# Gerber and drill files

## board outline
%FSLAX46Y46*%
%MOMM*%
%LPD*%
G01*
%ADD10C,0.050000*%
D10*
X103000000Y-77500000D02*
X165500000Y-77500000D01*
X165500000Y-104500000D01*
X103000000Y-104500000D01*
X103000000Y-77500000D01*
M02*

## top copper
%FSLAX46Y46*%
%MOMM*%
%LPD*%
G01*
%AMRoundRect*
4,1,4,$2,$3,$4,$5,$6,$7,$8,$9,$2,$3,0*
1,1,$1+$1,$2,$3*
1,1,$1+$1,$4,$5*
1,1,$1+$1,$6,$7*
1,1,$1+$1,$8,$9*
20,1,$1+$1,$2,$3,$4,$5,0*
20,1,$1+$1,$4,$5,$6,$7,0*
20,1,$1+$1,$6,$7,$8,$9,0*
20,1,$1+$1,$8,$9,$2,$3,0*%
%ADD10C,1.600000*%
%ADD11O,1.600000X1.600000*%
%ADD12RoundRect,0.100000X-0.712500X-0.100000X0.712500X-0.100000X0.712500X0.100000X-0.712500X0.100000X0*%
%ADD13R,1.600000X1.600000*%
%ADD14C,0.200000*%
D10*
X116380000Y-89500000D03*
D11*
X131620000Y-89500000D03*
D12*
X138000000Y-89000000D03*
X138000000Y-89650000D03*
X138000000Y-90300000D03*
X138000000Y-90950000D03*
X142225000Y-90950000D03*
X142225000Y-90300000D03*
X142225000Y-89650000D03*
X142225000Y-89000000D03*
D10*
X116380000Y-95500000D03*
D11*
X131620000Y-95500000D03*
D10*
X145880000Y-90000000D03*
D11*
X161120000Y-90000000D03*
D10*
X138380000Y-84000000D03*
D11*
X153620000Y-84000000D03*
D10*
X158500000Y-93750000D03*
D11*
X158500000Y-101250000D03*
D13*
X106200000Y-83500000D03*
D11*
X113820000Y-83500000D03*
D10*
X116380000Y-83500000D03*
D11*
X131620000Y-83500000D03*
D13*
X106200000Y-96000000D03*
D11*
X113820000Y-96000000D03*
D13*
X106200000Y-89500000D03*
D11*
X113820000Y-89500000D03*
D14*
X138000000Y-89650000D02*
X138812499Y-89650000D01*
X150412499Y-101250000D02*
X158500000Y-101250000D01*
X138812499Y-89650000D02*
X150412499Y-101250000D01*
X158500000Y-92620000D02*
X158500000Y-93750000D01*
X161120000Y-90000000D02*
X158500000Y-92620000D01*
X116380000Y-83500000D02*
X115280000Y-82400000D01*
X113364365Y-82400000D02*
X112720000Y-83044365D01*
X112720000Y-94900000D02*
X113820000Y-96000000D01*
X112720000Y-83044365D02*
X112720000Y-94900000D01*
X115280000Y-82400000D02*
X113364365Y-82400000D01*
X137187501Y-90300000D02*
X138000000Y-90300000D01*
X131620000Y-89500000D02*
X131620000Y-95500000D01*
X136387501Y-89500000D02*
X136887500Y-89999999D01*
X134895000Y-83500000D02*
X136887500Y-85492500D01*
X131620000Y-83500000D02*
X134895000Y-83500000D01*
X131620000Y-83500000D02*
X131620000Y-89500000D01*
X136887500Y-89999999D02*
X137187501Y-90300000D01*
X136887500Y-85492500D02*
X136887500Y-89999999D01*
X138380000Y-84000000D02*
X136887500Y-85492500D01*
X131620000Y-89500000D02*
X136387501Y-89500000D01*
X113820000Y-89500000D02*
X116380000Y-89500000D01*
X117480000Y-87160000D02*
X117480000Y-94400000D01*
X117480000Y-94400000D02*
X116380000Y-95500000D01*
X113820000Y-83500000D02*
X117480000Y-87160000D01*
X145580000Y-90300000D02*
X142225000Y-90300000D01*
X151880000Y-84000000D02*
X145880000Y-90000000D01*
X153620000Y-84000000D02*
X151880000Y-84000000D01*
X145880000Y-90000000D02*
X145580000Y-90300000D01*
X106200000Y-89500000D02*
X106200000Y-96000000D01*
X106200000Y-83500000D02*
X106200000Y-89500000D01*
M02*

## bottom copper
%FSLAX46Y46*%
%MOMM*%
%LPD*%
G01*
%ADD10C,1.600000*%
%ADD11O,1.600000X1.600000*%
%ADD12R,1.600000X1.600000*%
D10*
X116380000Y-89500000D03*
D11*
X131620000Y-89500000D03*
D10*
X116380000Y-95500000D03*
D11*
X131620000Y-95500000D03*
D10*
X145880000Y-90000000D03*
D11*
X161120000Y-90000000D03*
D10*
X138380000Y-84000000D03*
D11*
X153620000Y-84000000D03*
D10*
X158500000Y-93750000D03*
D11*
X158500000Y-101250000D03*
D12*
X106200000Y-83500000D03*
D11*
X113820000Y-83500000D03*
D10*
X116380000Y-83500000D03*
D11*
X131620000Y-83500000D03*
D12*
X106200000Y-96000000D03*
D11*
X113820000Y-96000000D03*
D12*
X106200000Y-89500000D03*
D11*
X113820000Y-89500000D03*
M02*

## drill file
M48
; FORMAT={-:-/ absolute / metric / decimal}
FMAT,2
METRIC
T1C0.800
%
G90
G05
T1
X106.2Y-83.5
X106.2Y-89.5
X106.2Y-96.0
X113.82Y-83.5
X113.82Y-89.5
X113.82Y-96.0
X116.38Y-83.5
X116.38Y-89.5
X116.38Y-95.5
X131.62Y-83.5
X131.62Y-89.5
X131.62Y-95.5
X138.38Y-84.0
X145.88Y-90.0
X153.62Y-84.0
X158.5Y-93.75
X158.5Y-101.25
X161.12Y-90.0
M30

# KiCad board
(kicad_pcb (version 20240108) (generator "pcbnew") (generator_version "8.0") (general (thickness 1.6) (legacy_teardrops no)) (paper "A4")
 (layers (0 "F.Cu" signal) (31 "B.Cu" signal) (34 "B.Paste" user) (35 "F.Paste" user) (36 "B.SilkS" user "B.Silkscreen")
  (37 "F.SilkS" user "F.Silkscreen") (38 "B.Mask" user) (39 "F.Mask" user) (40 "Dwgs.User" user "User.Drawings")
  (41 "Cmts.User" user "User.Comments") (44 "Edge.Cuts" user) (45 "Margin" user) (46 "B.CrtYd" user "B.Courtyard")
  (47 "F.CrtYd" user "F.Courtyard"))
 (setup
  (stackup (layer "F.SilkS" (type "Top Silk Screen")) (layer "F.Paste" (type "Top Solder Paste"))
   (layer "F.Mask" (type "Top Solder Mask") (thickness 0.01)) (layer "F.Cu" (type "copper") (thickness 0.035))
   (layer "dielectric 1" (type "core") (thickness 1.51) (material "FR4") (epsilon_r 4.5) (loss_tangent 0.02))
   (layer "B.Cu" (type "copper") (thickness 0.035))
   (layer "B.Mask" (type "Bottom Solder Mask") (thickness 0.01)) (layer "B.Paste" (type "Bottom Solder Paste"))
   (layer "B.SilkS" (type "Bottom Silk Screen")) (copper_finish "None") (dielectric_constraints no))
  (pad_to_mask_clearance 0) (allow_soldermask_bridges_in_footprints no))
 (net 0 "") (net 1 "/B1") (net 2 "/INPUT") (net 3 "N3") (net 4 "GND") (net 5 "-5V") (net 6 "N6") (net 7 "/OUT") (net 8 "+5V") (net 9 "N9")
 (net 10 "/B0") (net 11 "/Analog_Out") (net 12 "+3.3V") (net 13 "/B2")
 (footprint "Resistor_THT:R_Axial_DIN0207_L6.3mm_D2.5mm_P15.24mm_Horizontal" (layer "F.Cu") (at 116.38 89.5)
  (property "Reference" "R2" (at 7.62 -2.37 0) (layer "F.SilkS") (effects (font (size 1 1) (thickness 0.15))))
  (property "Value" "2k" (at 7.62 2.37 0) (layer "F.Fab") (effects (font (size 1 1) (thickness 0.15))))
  (pad "1" thru_hole circle (at 0 0) (size 1.6 1.6) (drill 0.8) (layers "*.Cu" "*.Mask") (remove_unused_layers no) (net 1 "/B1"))
  (pad "2" thru_hole oval (at 15.24 0) (size 1.6 1.6) (drill 0.8) (layers "*.Cu" "*.Mask") (remove_unused_layers no) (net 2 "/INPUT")))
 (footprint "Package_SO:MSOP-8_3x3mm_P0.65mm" (layer "F.Cu") (at 140.1125 89.975)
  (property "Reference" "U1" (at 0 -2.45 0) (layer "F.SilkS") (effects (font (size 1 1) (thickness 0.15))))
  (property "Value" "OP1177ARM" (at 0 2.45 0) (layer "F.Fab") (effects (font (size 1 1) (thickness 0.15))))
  (pad "1" smd roundrect (at -2.1125 -0.975) (size 1.625 0.4) (layers "F.Cu" "F.Paste" "F.Mask") (roundrect_rratio 0.25) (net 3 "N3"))
  (pad "2" smd roundrect (at -2.1125 -0.325) (size 1.625 0.4) (layers "F.Cu" "F.Paste" "F.Mask") (roundrect_rratio 0.25) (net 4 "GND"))
  (pad "3" smd roundrect (at -2.1125 0.325) (size 1.625 0.4) (layers "F.Cu" "F.Paste" "F.Mask") (roundrect_rratio 0.25) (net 2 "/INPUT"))
  (pad "4" smd roundrect (at -2.1125 0.975) (size 1.625 0.4) (layers "F.Cu" "F.Paste" "F.Mask") (roundrect_rratio 0.25) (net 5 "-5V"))
  (pad "5" smd roundrect (at 2.1125 0.975) (size 1.625 0.4) (layers "F.Cu" "F.Paste" "F.Mask") (roundrect_rratio 0.25) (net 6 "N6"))
  (pad "6" smd roundrect (at 2.1125 0.325) (size 1.625 0.4) (layers "F.Cu" "F.Paste" "F.Mask") (roundrect_rratio 0.25) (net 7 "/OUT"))
  (pad "7" smd roundrect (at 2.1125 -0.325) (size 1.625 0.4) (layers "F.Cu" "F.Paste" "F.Mask") (roundrect_rratio 0.25) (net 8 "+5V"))
  (pad "8" smd roundrect (at 2.1125 -0.975) (size 1.625 0.4) (layers "F.Cu" "F.Paste" "F.Mask") (roundrect_rratio 0.25) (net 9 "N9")))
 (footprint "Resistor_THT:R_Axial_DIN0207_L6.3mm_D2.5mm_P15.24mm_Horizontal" (layer "F.Cu") (at 116.38 95.5)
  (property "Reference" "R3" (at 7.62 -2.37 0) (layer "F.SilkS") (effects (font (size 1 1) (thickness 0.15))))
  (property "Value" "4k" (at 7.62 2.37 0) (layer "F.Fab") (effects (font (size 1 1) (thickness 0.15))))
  (pad "1" thru_hole circle (at 0 0) (size 1.6 1.6) (drill 0.8) (layers "*.Cu" "*.Mask") (remove_unused_layers no) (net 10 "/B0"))
  (pad "2" thru_hole oval (at 15.24 0) (size 1.6 1.6) (drill 0.8) (layers "*.Cu" "*.Mask") (remove_unused_layers no) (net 2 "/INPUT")))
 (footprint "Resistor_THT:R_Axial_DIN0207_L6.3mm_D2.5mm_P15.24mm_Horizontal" (layer "F.Cu") (at 145.88 90)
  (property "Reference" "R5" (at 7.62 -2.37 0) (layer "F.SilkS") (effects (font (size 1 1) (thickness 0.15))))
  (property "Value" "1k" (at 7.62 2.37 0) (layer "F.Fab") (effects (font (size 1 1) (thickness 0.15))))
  (pad "1" thru_hole circle (at 0 0) (size 1.6 1.6) (drill 0.8) (layers "*.Cu" "*.Mask") (remove_unused_layers no) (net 7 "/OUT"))
  (pad "2" thru_hole oval (at 15.24 0) (size 1.6 1.6) (drill 0.8) (layers "*.Cu" "*.Mask") (remove_unused_layers no) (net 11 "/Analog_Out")))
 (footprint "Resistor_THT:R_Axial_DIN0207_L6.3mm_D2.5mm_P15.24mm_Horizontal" (layer "F.Cu") (at 138.38 84)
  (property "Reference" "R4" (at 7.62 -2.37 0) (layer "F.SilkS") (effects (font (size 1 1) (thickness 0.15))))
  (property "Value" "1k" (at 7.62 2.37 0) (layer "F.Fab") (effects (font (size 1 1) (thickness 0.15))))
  (pad "1" thru_hole circle (at 0 0) (size 1.6 1.6) (drill 0.8) (layers "*.Cu" "*.Mask") (remove_unused_layers no) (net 2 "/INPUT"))
  (pad "2" thru_hole oval (at 15.24 0) (size 1.6 1.6) (drill 0.8) (layers "*.Cu" "*.Mask") (remove_unused_layers no) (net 7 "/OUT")))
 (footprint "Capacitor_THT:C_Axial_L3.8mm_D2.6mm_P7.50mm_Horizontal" (layer "F.Cu") (at 158.5 93.75 -90)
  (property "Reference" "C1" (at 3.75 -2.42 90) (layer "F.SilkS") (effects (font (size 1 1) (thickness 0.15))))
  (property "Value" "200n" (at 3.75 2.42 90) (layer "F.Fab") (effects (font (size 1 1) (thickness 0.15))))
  (pad "1" thru_hole circle (at 0 0 270) (size 1.6 1.6) (drill 0.8) (layers "*.Cu" "*.Mask") (remove_unused_layers no)
   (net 11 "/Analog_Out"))
  (pad "2" thru_hole oval (at 7.5 0 270) (size 1.6 1.6) (drill 0.8) (layers "*.Cu" "*.Mask") (remove_unused_layers no) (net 4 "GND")))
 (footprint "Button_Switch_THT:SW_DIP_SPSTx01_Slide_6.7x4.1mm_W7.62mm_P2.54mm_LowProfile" (layer "F.Cu") (at 106.2 83.5)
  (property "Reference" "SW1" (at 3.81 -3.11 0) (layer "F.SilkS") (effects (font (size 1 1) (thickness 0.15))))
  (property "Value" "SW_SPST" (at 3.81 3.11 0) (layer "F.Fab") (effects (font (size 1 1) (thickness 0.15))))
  (pad "1" thru_hole rect (at 0 0) (size 1.6 1.6) (drill 0.8) (layers "*.Cu" "*.Mask") (remove_unused_layers no) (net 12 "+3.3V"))
  (pad "2" thru_hole oval (at 7.62 0) (size 1.6 1.6) (drill 0.8) (layers "*.Cu" "*.Mask") (remove_unused_layers no) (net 10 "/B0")))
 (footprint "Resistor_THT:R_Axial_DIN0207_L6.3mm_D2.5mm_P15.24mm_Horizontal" (layer "F.Cu") (at 116.38 83.5)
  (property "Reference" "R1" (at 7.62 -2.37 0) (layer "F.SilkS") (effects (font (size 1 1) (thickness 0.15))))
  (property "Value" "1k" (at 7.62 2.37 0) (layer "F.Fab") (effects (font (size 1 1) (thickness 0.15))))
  (pad "1" thru_hole circle (at 0 0) (size 1.6 1.6) (drill 0.8) (layers "*.Cu" "*.Mask") (remove_unused_layers no) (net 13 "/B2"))
  (pad "2" thru_hole oval (at 15.24 0) (size 1.6 1.6) (drill 0.8) (layers "*.Cu" "*.Mask") (remove_unused_layers no) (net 2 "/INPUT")))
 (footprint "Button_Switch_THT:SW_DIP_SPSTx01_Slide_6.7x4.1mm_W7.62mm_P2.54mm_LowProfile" (layer "F.Cu") (at 106.2 96)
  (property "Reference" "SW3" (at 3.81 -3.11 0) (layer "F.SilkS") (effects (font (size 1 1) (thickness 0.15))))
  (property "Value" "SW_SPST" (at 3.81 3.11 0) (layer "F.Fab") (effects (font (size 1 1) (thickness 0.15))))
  (pad "1" thru_hole rect (at 0 0) (size 1.6 1.6) (drill 0.8) (layers "*.Cu" "*.Mask") (remove_unused_layers no) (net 12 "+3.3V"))
  (pad "2" thru_hole oval (at 7.62 0) (size 1.6 1.6) (drill 0.8) (layers "*.Cu" "*.Mask") (remove_unused_layers no) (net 13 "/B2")))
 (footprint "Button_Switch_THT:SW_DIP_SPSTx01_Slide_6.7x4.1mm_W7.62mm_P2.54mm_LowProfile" (layer "F.Cu") (at 106.2 89.5)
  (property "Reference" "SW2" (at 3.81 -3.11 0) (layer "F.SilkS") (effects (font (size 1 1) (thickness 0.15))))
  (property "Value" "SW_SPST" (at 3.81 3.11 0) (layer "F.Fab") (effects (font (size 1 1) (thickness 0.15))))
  (pad "1" thru_hole rect (at 0 0) (size 1.6 1.6) (drill 0.8) (layers "*.Cu" "*.Mask") (remove_unused_layers no) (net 12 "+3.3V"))
  (pad "2" thru_hole oval (at 7.62 0) (size 1.6 1.6) (drill 0.8) (layers "*.Cu" "*.Mask") (remove_unused_layers no) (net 1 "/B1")))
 (gr_rect (start 103 77.5) (end 165.5 104.5) (stroke (width 0.05) (type default)) (fill none) (layer "Edge.Cuts"))
 (segment (start 138 89.65) (end 138.812499 89.65) (width 0.2) (layer "F.Cu") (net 4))
 (segment (start 150.412499 101.25) (end 158.5 101.25) (width 0.2) (layer "F.Cu") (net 4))
 (segment (start 138.812499 89.65) (end 150.412499 101.25) (width 0.2) (layer "F.Cu") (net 4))
 (segment (start 158.5 92.62) (end 158.5 93.75) (width 0.2) (layer "F.Cu") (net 11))
 (segment (start 161.12 90) (end 158.5 92.62) (width 0.2) (layer "F.Cu") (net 11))
 (segment (start 116.38 83.5) (end 115.28 82.4) (width 0.2) (layer "F.Cu") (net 13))
 (segment (start 113.364365 82.4) (end 112.72 83.044365) (width 0.2) (layer "F.Cu") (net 13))
 (segment (start 112.72 94.9) (end 113.82 96) (width 0.2) (layer "F.Cu") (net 13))
 (segment (start 112.72 83.044365) (end 112.72 94.9) (width 0.2) (layer "F.Cu") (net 13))
 (segment (start 115.28 82.4) (end 113.364365 82.4) (width 0.2) (layer "F.Cu") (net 13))
 (segment (start 137.187501 90.3) (end 138 90.3) (width 0.2) (layer "F.Cu") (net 2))
 (segment (start 131.62 89.5) (end 131.62 95.5) (width 0.2) (layer "F.Cu") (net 2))
 (segment (start 136.387501 89.5) (end 136.8875 89.999999) (width 0.2) (layer "F.Cu") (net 2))
 (segment (start 134.895 83.5) (end 136.8875 85.4925) (width 0.2) (layer "F.Cu") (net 2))
 (segment (start 131.62 83.5) (end 134.895 83.5) (width 0.2) (layer "F.Cu") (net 2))
 (segment (start 131.62 83.5) (end 131.62 89.5) (width 0.2) (layer "F.Cu") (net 2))
 (segment (start 136.8875 89.999999) (end 137.187501 90.3) (width 0.2) (layer "F.Cu") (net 2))
 (segment (start 136.8875 85.4925) (end 136.8875 89.999999) (width 0.2) (layer "F.Cu") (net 2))
 (segment (start 138.38 84) (end 136.8875 85.4925) (width 0.2) (layer "F.Cu") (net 2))
 (segment (start 131.62 89.5) (end 136.387501 89.5) (width 0.2) (layer "F.Cu") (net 2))
 (segment (start 113.82 89.5) (end 116.38 89.5) (width 0.2) (layer "F.Cu") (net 1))
 (segment (start 117.48 87.16) (end 117.48 94.4) (width 0.2) (layer "F.Cu") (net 10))
 (segment (start 117.48 94.4) (end 116.38 95.5) (width 0.2) (layer "F.Cu") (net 10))
 (segment (start 113.82 83.5) (end 117.48 87.16) (width 0.2) (layer "F.Cu") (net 10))
 (segment (start 145.58 90.3) (end 142.225 90.3) (width 0.2) (layer "F.Cu") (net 7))
 (segment (start 151.88 84) (end 145.88 90) (width 0.2) (layer "F.Cu") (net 7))
 (segment (start 153.62 84) (end 151.88 84) (width 0.2) (layer "F.Cu") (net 7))
 (segment (start 145.88 90) (end 145.58 90.3) (width 0.2) (layer "F.Cu") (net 7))
 (segment (start 106.2 89.5) (end 106.2 96) (width 0.2) (layer "F.Cu") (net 12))
 (segment (start 106.2 83.5) (end 106.2 89.5) (width 0.2) (layer "F.Cu") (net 12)))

